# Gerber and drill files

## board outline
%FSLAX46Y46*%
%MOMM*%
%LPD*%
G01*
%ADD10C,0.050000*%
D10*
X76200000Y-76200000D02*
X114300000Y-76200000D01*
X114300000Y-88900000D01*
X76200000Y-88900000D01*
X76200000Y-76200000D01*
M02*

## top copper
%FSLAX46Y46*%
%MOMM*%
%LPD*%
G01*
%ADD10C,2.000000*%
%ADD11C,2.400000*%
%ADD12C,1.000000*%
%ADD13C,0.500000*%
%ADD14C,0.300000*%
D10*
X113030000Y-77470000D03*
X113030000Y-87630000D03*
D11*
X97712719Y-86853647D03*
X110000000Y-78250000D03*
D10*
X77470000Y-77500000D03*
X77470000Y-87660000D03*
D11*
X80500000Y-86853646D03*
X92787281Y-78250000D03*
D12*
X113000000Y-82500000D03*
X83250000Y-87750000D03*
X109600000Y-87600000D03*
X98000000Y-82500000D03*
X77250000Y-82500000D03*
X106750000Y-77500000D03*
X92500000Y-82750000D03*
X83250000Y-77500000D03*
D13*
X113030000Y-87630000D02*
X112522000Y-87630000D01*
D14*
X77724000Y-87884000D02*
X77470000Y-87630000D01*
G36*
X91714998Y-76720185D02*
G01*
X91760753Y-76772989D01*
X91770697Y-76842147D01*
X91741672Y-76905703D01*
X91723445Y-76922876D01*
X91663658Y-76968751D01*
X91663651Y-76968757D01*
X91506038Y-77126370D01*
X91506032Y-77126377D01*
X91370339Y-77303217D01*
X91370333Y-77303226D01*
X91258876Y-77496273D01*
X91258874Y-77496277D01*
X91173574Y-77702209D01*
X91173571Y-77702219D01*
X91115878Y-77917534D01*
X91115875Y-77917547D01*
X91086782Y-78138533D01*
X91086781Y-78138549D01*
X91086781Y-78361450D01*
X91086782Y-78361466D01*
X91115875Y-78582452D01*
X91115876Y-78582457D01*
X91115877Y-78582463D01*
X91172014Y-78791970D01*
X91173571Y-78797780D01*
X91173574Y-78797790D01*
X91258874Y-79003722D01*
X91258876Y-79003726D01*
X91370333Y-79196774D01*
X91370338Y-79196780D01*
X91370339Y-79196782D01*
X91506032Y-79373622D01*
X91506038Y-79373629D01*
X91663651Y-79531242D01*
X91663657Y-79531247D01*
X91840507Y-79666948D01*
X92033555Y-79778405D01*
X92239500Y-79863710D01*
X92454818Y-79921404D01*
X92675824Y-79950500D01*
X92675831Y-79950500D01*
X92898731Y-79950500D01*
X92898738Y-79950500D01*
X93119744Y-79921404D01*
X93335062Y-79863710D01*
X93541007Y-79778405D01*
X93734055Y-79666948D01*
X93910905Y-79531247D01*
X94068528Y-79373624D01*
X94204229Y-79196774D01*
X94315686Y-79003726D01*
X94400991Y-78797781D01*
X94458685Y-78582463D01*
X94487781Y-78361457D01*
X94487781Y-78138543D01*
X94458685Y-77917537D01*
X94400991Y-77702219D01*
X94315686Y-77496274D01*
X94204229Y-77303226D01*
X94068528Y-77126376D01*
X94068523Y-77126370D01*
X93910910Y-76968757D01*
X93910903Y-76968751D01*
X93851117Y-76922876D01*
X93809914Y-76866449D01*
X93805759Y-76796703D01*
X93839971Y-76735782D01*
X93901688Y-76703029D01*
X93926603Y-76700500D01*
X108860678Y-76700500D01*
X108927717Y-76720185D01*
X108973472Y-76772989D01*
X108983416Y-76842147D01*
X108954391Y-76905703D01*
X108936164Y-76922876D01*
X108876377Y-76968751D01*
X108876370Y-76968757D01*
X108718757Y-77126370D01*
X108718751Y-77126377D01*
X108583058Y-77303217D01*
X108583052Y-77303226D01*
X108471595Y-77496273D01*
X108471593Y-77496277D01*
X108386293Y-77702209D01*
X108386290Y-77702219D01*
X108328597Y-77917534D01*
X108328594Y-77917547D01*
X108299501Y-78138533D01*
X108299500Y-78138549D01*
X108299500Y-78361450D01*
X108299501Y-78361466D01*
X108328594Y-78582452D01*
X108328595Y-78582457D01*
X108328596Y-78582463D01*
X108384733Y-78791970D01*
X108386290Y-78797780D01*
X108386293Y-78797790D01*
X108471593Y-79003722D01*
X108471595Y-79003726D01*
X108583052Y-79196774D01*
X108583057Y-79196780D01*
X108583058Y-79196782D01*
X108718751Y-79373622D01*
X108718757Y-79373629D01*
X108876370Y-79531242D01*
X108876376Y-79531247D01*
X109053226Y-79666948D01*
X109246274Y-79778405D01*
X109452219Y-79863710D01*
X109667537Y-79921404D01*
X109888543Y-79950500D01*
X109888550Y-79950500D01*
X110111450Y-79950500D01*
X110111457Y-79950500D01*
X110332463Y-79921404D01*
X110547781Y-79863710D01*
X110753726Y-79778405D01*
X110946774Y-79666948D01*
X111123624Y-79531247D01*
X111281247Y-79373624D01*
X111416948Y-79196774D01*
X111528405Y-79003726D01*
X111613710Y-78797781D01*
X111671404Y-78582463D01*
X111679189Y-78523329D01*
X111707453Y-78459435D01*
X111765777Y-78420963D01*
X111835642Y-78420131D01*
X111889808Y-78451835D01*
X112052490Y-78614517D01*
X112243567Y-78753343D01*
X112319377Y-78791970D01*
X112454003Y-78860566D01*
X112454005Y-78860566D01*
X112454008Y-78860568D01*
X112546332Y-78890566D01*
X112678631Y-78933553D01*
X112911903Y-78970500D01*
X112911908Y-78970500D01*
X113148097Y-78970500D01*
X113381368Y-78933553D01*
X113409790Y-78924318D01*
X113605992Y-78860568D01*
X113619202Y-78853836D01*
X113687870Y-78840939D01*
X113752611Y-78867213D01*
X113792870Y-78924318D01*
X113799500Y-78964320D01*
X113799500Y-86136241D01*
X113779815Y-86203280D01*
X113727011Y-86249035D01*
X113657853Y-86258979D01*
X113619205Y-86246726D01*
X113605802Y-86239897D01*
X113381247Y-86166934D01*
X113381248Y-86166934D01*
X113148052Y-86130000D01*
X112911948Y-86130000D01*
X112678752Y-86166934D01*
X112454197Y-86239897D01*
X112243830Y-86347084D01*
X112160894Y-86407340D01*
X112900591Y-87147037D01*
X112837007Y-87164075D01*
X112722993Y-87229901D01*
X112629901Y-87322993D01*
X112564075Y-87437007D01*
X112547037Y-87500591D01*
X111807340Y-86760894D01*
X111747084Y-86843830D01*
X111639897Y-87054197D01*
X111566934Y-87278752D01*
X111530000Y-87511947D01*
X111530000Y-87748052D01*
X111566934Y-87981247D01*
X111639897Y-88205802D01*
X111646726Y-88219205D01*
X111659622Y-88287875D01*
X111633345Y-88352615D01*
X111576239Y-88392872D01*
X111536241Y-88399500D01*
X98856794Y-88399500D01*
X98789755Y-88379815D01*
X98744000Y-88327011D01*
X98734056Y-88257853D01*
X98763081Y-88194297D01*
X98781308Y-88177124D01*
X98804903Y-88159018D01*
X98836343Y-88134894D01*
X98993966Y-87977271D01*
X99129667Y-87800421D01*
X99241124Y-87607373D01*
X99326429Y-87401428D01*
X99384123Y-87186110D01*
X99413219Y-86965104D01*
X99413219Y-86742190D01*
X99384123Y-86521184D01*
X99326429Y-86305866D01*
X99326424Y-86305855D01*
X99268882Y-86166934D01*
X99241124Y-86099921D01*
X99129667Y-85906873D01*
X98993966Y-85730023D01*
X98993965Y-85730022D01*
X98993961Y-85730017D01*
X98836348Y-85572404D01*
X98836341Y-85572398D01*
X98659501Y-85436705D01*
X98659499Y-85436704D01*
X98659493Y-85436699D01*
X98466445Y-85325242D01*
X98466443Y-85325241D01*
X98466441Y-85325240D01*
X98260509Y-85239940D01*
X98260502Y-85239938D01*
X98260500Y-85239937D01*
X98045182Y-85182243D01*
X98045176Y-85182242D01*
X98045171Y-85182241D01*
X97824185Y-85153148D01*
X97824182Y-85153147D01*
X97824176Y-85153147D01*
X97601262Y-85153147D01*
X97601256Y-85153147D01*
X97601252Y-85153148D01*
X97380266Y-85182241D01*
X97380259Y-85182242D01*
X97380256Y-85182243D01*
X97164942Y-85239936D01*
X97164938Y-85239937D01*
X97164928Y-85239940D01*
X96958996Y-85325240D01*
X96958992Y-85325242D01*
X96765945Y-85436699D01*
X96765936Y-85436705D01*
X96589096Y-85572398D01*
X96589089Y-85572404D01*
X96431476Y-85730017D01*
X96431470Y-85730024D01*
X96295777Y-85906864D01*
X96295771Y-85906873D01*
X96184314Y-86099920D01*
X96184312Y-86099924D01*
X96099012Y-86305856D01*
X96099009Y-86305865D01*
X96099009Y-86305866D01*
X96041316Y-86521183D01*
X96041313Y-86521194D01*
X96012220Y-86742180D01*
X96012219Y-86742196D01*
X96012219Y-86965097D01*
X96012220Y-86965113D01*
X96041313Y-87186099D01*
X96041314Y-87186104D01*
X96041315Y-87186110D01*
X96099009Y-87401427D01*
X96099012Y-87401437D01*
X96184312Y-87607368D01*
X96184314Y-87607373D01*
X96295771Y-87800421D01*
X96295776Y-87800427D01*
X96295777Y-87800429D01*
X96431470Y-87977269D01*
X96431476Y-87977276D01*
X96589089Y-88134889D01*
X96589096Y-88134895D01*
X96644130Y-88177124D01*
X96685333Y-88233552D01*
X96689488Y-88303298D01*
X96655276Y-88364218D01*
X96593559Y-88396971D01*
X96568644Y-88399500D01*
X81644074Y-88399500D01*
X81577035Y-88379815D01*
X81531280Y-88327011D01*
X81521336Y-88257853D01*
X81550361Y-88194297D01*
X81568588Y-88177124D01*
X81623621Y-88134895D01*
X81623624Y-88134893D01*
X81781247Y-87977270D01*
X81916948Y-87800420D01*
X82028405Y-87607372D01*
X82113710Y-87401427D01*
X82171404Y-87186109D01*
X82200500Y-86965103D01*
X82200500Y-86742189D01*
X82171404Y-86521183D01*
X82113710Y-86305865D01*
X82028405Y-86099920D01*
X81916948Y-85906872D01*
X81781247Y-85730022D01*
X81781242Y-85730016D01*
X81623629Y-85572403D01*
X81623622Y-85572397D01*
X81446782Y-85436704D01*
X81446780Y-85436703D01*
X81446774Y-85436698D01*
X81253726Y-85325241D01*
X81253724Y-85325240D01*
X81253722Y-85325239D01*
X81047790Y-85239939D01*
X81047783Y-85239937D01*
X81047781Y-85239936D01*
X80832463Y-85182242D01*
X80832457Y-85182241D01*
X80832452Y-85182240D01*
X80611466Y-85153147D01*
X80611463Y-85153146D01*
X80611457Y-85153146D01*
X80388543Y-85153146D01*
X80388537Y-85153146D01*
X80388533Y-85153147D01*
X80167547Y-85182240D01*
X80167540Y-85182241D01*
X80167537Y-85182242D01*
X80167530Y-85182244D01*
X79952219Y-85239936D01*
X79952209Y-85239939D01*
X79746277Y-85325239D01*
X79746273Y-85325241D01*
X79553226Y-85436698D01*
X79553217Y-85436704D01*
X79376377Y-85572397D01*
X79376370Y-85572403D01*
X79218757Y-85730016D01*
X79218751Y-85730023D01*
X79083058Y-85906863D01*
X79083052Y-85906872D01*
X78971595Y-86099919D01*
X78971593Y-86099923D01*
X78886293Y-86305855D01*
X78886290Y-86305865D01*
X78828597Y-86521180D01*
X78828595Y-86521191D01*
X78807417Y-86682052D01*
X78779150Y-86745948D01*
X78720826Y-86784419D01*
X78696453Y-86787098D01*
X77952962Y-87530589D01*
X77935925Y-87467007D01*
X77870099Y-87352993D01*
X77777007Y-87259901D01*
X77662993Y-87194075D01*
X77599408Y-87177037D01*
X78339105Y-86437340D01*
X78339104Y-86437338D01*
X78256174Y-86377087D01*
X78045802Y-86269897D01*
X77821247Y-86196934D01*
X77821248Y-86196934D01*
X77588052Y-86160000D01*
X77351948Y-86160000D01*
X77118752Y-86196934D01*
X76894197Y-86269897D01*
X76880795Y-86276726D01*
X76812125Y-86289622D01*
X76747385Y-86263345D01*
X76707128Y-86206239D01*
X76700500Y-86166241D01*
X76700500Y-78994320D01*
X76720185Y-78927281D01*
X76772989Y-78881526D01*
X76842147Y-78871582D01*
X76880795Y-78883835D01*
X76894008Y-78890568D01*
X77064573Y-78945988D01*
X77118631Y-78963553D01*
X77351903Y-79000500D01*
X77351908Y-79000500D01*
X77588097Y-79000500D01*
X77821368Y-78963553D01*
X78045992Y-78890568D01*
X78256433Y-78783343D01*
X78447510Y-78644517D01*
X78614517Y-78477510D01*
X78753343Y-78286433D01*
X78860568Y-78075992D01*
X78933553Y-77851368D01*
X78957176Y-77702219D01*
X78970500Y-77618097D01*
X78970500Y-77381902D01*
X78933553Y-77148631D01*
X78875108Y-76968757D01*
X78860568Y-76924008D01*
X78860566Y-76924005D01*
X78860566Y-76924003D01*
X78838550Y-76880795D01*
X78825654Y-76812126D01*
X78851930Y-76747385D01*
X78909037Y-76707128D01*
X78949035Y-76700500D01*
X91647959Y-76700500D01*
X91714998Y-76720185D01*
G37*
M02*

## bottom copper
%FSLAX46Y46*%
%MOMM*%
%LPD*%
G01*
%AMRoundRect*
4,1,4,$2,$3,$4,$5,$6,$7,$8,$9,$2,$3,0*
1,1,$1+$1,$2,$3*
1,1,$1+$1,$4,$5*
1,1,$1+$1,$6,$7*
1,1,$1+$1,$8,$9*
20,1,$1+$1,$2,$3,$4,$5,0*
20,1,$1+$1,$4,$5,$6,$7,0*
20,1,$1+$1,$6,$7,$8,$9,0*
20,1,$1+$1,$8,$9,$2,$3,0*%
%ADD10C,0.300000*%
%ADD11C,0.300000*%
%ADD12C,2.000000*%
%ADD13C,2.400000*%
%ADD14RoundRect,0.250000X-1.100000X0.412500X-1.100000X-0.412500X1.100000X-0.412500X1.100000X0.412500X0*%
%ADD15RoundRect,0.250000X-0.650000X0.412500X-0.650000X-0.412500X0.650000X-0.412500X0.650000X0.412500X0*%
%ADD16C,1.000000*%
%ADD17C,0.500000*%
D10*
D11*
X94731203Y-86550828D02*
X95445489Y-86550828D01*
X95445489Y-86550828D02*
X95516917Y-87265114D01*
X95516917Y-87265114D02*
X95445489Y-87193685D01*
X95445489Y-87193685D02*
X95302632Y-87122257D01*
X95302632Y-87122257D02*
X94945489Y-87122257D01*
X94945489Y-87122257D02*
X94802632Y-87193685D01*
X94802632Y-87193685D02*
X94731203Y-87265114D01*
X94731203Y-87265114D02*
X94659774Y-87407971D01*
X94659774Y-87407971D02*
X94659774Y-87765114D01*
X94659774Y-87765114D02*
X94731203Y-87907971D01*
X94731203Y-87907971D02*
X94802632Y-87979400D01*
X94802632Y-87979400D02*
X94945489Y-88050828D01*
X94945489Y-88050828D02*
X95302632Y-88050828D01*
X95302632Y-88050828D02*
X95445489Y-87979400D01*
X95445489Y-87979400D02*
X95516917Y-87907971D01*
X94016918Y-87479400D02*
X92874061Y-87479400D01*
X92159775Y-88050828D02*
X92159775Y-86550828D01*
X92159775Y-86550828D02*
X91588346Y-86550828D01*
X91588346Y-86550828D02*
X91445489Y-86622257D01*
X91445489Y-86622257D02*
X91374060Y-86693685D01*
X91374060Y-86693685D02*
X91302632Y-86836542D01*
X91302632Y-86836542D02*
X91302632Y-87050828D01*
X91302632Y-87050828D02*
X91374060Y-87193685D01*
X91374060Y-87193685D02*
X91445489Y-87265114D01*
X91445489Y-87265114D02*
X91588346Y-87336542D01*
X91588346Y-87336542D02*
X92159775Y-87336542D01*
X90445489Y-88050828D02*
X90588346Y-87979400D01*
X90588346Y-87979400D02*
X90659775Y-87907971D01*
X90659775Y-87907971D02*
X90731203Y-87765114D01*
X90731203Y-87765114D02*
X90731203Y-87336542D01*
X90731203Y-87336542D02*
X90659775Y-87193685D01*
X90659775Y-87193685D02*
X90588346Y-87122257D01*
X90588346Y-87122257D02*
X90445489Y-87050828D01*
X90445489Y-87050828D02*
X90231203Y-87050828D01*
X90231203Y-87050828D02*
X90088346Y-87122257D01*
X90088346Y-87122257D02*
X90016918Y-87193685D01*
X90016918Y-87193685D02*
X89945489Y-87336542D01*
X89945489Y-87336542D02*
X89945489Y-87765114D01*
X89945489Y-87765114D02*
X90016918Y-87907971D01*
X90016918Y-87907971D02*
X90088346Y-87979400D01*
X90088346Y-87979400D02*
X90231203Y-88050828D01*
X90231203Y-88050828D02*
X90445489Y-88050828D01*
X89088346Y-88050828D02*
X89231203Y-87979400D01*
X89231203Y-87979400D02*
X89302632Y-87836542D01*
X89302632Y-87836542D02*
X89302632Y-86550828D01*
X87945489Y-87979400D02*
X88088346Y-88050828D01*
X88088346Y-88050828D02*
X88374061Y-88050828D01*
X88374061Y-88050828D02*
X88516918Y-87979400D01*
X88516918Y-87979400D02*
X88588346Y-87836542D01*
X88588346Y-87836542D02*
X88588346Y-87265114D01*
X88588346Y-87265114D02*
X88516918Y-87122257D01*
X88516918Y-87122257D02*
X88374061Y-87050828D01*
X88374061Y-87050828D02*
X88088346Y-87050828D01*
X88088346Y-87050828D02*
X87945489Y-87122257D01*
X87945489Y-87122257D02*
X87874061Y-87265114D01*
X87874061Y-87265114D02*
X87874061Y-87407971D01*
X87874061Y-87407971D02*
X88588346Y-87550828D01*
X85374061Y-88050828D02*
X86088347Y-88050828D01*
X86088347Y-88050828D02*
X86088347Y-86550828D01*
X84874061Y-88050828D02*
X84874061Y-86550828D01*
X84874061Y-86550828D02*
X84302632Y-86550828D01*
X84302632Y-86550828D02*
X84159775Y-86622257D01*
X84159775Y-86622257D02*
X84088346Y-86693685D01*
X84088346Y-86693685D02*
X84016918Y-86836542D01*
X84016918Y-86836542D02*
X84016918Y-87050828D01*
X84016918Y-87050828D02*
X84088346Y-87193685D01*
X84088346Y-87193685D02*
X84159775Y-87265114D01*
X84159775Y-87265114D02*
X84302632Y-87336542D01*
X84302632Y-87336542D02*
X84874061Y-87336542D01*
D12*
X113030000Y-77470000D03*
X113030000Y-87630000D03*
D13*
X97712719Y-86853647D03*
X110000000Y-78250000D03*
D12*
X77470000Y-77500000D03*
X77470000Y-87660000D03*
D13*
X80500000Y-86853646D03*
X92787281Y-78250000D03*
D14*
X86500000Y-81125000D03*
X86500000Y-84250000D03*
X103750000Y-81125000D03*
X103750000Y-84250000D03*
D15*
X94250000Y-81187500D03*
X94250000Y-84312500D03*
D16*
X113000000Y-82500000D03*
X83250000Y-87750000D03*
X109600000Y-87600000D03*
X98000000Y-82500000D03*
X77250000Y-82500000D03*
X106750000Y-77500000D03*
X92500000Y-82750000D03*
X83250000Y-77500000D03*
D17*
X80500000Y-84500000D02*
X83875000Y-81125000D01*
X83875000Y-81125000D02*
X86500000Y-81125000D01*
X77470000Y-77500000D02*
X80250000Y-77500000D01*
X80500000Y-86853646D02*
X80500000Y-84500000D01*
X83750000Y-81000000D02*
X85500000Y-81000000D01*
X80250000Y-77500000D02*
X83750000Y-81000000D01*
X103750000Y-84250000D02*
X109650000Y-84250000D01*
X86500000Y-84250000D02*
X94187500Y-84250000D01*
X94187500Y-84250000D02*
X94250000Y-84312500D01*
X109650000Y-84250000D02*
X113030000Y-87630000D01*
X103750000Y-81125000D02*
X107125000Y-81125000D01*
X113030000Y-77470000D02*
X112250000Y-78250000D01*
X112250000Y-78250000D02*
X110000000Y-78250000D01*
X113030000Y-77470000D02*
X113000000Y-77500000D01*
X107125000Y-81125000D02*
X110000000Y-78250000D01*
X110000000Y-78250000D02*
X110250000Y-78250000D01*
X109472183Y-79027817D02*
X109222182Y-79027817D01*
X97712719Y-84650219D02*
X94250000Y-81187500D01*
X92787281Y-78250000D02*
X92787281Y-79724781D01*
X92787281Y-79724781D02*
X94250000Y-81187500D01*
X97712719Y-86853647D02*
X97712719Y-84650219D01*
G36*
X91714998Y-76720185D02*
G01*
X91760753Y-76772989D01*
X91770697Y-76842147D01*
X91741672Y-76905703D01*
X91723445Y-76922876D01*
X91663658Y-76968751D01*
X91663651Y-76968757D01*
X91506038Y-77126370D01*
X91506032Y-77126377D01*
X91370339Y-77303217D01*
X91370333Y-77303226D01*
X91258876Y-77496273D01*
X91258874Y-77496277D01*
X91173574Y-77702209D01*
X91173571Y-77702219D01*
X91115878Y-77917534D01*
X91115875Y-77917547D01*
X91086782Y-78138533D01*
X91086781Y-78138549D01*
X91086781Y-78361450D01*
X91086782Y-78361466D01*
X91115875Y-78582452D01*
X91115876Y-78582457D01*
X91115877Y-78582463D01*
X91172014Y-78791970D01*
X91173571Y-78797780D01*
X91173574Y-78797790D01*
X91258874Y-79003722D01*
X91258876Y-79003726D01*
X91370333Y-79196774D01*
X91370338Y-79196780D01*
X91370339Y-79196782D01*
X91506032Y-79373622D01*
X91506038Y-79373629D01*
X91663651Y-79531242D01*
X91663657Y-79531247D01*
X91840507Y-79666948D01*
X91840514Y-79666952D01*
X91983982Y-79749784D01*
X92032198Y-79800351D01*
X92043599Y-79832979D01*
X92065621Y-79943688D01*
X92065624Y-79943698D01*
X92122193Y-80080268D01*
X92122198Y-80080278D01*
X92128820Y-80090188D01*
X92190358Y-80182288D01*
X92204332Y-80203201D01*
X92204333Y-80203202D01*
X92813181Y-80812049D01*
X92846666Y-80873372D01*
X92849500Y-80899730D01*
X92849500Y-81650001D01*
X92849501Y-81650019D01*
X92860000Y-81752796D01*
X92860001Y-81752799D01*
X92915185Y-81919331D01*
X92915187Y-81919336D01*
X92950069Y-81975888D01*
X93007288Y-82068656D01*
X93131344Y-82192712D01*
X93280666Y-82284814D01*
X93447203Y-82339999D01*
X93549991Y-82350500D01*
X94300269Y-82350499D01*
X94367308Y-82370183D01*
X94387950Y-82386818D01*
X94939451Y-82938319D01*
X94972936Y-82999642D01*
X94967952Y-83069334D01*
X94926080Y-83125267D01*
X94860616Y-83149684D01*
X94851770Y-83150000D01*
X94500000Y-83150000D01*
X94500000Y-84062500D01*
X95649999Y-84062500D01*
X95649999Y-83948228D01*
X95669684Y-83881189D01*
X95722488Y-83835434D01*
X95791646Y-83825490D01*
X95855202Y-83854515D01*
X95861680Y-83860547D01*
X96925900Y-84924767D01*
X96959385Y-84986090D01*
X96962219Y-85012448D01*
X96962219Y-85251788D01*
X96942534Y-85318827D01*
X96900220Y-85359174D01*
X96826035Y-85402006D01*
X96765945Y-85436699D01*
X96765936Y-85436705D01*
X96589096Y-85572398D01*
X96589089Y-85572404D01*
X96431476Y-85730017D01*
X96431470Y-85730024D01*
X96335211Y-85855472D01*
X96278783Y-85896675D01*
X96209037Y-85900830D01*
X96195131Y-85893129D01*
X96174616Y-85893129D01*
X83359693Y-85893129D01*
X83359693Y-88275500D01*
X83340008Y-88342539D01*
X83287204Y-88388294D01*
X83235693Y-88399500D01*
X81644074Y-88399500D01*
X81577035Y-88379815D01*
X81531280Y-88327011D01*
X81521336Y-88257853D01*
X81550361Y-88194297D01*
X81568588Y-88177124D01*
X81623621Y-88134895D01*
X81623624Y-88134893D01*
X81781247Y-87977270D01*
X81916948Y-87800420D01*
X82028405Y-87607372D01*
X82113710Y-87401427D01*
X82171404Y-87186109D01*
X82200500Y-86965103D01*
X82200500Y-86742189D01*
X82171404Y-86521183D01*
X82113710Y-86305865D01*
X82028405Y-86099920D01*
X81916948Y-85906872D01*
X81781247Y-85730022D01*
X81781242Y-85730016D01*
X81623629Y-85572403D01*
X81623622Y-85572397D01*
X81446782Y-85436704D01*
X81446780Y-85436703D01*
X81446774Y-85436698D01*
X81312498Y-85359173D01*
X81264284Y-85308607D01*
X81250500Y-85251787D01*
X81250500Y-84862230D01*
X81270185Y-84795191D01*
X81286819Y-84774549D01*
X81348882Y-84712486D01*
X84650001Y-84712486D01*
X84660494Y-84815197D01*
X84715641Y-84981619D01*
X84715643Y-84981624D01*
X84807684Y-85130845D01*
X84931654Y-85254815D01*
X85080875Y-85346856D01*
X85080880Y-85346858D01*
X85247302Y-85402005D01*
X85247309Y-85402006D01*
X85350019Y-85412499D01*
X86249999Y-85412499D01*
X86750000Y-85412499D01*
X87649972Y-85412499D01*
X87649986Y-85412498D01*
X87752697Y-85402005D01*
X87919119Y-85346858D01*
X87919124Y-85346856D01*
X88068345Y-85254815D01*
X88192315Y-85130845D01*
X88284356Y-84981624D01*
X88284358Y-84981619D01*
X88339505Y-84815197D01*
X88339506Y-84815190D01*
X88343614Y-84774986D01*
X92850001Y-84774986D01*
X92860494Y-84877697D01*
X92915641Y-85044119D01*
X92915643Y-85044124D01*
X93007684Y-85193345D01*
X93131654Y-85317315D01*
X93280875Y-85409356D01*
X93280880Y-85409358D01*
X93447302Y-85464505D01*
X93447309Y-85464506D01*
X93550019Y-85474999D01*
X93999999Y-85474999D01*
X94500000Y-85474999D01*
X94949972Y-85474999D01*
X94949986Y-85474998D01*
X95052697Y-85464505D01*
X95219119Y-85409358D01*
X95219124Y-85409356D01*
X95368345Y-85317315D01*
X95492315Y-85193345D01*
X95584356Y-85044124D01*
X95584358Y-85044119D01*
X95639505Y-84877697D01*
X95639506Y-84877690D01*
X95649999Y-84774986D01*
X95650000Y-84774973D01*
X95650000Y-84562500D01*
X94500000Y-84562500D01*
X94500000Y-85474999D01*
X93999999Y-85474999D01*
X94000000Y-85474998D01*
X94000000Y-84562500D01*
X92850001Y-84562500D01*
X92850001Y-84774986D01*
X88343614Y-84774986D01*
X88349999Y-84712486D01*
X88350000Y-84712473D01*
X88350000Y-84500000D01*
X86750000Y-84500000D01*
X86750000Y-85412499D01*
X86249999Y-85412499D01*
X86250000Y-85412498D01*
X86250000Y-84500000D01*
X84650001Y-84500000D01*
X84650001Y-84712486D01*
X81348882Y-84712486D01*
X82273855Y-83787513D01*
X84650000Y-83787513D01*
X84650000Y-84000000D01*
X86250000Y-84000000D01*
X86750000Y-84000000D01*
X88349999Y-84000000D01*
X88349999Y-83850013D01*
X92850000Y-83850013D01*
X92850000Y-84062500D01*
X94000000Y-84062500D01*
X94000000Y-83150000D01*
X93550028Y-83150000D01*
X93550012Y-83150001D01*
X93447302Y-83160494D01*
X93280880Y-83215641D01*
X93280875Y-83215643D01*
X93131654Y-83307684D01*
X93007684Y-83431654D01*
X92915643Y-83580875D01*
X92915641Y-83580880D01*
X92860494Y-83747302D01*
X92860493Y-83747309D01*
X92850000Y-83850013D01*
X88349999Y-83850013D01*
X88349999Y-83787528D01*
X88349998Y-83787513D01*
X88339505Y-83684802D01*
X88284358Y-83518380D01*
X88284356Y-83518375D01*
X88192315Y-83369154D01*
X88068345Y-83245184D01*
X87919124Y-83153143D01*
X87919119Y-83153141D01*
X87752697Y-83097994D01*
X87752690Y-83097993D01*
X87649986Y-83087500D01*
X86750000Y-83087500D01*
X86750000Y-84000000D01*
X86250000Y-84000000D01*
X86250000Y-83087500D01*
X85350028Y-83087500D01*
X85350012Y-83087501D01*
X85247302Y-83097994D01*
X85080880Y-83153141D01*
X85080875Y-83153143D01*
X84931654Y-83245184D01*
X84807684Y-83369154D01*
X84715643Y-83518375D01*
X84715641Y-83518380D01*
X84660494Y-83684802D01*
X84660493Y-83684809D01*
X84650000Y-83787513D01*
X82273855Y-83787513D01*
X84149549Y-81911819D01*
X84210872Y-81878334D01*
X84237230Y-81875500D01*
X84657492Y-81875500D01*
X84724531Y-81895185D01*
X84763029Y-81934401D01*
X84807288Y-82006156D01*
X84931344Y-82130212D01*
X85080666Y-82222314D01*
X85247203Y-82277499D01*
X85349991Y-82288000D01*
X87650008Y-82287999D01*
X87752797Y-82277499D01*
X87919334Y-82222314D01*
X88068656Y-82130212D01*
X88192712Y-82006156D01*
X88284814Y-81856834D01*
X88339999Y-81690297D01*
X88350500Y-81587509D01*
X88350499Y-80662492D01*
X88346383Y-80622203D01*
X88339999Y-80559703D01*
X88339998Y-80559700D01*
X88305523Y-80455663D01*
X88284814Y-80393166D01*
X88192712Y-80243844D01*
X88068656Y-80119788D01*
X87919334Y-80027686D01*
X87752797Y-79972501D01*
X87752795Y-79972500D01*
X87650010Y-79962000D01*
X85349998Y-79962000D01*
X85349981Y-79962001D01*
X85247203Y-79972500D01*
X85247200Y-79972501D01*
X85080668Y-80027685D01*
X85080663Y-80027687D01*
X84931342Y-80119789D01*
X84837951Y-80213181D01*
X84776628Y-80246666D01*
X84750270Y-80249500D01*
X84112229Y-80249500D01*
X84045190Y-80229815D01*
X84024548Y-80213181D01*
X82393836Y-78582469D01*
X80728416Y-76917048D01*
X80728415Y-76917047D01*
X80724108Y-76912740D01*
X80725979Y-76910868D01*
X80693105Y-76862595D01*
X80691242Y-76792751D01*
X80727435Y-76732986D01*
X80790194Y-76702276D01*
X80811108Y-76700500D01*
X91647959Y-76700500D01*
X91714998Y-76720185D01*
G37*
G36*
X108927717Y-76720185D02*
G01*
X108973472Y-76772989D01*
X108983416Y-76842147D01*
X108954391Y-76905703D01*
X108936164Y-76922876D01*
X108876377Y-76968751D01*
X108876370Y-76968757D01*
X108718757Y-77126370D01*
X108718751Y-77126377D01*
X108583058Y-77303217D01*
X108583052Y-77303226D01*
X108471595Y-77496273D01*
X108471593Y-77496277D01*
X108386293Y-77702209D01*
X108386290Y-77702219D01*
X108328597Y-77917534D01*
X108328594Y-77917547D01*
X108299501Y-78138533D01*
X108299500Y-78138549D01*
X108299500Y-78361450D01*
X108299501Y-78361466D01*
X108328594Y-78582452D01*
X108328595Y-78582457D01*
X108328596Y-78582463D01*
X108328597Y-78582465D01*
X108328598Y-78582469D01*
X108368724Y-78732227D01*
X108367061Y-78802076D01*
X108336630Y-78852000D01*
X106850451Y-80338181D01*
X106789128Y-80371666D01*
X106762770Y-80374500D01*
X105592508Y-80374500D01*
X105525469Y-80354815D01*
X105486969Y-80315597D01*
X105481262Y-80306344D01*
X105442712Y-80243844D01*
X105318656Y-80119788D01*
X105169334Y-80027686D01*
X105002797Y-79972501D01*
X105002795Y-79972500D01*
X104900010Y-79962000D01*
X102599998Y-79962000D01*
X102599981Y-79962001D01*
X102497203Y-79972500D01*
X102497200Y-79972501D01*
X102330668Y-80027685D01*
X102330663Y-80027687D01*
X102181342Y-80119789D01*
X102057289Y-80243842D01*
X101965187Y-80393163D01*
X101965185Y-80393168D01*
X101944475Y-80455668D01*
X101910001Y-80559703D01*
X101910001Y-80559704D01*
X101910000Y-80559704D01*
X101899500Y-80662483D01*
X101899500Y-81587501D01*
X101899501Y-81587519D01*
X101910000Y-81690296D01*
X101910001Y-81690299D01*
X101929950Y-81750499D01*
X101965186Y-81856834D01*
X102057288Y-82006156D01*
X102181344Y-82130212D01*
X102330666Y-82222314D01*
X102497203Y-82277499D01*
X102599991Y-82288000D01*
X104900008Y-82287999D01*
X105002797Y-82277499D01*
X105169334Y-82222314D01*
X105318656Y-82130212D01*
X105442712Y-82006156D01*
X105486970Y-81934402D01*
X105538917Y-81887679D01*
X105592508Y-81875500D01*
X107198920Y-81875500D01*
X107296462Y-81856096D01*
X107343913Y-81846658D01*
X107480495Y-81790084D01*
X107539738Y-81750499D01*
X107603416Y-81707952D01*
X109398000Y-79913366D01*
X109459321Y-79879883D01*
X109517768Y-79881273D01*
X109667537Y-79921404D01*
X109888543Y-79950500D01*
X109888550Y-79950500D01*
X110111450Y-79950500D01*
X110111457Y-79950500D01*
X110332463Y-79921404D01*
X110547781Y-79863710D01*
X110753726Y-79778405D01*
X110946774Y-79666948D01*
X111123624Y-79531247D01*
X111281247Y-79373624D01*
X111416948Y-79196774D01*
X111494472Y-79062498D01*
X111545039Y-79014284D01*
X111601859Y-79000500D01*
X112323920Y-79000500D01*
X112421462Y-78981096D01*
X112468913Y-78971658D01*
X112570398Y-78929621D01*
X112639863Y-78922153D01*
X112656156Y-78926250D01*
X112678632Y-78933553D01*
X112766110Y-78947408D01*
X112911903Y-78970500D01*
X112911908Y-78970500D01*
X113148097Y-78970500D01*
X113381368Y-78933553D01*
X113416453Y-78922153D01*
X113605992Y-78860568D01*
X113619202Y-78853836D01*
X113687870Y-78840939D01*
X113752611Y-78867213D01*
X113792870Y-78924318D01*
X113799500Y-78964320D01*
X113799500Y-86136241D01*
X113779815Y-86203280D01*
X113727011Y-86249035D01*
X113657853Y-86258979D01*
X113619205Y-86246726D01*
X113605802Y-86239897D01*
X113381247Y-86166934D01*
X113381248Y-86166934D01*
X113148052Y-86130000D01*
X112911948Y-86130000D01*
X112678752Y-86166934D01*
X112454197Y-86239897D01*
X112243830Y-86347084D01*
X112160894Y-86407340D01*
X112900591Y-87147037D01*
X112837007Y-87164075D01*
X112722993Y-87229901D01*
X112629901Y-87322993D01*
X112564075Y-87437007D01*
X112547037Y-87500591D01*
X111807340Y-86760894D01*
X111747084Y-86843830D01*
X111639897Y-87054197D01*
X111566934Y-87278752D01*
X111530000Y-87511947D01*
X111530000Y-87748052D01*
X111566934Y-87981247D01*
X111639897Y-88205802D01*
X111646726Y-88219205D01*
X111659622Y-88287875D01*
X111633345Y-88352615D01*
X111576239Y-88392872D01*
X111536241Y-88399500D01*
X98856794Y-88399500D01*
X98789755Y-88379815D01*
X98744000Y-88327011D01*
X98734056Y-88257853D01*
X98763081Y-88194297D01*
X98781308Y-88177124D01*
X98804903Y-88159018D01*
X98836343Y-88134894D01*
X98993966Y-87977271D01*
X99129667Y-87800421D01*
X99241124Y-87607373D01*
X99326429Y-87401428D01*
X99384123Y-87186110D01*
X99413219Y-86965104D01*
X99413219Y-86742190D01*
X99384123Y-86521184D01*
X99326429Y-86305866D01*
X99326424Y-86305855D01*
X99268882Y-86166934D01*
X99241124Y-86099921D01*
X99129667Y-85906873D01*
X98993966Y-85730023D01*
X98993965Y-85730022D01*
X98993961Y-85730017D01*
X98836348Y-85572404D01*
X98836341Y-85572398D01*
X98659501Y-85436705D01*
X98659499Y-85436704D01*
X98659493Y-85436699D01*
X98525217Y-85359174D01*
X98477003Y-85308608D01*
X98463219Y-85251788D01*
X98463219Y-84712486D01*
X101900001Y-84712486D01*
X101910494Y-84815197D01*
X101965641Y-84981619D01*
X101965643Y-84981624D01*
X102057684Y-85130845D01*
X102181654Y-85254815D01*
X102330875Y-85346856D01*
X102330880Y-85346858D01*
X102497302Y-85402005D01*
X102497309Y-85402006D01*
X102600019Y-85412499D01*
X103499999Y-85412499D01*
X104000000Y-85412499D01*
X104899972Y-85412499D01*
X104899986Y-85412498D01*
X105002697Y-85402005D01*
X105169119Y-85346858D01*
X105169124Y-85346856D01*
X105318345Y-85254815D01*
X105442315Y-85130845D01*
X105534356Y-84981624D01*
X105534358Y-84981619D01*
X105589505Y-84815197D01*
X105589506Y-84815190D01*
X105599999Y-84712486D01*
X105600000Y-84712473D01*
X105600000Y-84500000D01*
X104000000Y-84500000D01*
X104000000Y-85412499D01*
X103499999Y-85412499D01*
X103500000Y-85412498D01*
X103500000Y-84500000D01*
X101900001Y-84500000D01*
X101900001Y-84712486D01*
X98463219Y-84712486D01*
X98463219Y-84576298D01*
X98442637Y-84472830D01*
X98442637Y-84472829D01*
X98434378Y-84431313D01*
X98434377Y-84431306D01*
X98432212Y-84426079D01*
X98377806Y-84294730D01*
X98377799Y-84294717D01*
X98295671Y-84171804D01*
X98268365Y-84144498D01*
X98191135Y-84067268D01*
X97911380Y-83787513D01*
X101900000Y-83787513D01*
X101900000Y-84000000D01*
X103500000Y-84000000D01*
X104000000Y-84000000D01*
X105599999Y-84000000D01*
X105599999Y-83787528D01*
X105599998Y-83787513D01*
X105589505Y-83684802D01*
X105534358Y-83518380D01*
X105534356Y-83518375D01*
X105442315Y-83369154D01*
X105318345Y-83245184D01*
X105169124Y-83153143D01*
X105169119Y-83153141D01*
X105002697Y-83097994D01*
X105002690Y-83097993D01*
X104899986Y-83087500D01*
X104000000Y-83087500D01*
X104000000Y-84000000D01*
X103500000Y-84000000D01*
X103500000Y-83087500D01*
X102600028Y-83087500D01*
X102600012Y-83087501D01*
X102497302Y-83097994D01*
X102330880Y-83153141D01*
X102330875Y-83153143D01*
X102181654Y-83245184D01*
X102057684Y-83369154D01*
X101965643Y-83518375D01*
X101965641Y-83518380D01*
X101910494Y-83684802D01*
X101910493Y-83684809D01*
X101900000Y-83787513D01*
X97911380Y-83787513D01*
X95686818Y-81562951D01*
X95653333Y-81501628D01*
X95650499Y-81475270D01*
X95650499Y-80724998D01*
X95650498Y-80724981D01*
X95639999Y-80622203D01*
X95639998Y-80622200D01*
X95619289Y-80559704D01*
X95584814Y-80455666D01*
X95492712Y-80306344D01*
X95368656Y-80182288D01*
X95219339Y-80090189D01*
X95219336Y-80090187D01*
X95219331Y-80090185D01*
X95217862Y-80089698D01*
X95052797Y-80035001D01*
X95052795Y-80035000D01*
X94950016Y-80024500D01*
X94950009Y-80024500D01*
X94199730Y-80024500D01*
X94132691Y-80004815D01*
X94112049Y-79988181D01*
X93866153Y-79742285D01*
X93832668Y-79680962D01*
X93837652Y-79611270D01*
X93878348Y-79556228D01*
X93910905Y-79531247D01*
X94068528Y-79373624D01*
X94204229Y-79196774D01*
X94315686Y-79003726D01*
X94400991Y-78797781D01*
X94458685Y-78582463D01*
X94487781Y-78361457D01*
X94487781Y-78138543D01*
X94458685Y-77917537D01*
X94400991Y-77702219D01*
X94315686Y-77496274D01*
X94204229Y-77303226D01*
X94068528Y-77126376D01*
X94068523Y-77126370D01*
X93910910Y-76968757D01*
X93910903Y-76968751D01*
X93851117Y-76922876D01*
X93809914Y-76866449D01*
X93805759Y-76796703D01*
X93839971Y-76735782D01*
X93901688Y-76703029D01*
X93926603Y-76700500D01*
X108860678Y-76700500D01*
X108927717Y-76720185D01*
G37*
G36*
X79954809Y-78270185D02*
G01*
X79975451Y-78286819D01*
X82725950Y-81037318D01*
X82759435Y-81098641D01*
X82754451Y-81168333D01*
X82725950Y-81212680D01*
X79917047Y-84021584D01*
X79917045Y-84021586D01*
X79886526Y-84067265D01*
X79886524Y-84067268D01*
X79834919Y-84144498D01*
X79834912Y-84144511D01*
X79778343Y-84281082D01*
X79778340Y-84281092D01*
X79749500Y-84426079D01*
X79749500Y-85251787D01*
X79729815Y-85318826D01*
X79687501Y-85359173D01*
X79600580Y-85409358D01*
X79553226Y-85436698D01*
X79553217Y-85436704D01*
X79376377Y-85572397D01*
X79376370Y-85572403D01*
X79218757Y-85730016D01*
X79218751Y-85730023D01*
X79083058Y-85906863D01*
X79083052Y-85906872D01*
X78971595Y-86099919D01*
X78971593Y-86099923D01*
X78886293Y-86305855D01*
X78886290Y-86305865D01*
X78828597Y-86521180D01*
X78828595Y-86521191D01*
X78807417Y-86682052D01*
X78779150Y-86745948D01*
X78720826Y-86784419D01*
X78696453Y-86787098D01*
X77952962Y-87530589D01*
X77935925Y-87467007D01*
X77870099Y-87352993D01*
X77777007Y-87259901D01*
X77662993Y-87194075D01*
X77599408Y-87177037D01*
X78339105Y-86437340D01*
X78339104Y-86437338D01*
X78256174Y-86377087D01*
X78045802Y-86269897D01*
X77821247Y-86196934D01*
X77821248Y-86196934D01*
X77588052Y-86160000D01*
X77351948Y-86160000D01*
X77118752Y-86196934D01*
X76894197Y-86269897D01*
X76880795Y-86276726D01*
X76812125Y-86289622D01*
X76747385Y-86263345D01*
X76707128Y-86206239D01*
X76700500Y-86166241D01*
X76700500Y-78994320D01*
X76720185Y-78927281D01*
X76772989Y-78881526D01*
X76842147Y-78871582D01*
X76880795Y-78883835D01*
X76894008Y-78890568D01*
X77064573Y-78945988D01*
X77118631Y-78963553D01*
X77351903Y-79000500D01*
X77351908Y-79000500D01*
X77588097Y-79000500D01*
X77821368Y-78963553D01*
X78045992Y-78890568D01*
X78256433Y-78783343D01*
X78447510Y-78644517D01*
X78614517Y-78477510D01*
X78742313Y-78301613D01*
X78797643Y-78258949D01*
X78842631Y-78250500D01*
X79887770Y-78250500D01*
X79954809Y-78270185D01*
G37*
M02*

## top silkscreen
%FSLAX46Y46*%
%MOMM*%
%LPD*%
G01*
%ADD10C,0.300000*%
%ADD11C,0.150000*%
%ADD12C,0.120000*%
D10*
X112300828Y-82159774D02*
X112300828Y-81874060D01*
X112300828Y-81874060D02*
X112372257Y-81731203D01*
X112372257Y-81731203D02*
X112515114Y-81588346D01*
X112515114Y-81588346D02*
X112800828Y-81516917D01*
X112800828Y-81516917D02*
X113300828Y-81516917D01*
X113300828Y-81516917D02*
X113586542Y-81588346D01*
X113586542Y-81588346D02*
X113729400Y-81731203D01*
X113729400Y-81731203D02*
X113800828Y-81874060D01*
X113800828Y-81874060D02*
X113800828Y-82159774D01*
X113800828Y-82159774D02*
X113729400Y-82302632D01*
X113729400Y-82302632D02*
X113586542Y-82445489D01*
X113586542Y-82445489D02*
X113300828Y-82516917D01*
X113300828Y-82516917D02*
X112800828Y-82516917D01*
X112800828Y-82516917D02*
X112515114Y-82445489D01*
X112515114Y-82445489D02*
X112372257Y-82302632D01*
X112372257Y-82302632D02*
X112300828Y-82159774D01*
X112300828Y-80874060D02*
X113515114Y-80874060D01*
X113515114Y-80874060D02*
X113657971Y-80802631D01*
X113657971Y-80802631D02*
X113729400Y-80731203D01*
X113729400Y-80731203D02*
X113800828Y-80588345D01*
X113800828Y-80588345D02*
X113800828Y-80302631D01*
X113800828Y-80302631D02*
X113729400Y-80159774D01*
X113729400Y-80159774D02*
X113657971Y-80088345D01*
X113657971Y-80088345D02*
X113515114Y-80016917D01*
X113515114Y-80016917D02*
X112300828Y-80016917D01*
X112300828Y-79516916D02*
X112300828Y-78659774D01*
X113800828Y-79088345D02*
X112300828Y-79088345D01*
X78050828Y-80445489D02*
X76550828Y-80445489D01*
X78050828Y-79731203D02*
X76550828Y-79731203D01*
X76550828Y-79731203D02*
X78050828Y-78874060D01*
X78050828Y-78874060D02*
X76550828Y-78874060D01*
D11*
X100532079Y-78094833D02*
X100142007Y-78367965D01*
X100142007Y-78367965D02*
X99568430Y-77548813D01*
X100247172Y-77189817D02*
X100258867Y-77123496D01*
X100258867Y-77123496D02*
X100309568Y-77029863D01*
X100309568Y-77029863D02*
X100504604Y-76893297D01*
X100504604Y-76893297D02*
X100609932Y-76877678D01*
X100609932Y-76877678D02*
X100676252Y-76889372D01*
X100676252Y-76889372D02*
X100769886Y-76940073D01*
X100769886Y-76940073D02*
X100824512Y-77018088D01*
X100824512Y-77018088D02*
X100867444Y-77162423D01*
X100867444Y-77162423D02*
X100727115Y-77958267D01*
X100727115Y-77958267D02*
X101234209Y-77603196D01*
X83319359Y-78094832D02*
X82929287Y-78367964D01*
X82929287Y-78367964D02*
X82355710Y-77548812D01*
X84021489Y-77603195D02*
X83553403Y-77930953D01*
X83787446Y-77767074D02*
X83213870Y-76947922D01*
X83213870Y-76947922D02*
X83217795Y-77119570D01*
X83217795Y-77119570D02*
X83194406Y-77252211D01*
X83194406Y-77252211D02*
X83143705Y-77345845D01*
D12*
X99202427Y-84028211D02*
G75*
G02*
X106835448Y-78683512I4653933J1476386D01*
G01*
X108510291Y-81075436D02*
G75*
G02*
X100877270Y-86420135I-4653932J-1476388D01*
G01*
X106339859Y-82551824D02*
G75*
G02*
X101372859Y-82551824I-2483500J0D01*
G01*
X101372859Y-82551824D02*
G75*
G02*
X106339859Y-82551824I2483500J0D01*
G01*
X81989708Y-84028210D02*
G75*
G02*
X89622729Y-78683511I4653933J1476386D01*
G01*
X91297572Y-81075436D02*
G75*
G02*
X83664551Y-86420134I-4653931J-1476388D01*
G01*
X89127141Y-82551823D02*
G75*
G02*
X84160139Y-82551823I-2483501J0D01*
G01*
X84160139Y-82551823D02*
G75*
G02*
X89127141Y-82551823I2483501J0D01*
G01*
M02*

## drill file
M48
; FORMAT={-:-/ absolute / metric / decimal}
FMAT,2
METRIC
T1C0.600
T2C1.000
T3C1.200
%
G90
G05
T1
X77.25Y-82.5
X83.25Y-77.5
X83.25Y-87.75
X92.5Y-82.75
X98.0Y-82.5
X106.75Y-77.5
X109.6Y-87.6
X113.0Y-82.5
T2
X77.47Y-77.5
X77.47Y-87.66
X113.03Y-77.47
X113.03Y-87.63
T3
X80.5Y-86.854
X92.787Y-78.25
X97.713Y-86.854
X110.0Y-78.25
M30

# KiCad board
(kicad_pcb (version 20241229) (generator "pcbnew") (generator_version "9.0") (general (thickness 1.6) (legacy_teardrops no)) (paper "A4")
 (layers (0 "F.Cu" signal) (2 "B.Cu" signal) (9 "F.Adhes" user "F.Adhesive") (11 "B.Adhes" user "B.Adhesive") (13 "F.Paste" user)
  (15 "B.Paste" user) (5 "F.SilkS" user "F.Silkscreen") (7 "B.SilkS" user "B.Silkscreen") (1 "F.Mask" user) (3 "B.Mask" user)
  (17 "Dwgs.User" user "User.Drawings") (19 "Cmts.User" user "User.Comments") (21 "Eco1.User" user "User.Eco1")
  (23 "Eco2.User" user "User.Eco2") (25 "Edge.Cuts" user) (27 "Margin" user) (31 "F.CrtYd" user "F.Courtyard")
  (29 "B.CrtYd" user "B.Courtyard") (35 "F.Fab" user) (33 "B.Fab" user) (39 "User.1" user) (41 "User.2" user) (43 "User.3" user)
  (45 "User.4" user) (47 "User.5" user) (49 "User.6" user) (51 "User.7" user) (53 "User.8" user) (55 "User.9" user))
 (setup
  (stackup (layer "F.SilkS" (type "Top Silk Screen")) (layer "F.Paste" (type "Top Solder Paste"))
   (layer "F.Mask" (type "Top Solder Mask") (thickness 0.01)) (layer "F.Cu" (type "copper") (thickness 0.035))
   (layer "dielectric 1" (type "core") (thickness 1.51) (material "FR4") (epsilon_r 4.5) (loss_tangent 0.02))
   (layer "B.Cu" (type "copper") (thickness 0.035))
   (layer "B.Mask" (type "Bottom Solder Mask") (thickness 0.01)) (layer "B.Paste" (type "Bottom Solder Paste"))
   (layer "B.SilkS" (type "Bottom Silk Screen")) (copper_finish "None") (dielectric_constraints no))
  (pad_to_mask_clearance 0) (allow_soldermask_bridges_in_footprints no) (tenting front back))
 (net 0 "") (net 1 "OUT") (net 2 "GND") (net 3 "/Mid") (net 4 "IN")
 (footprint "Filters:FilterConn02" (layer "F.Cu") (at 113.03 82.55)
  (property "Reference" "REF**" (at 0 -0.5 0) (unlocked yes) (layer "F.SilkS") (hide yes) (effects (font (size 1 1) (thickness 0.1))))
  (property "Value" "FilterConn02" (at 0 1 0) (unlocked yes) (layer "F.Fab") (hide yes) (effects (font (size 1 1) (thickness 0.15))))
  (pad "3" thru_hole circle (at 0 -5.08) (size 2 2) (drill 1) (layers "*.Cu" "*.Mask") (remove_unused_layers no) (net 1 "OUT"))
  (pad "4" thru_hole circle (at 0 5.08) (size 2 2) (drill 1) (layers "*.Cu" "*.Mask") (remove_unused_layers no) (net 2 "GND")))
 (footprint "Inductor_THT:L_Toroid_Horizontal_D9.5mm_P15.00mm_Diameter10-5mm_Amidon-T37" (layer "F.Cu") (at 97.712719 86.853647 35)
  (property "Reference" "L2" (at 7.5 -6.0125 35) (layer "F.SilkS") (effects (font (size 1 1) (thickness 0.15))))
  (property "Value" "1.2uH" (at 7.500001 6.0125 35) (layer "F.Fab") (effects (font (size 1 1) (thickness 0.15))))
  (fp_arc (start 2.840901 -1.46) (mid 7.5 -4.882499) (end 12.159099 -1.46) (stroke (width 0.12) (type solid)) (layer "F.SilkS"))
  (fp_arc (start 12.159099 1.46) (mid 7.5 4.8825) (end 2.840901 1.46) (stroke (width 0.12) (type solid)) (layer "F.SilkS"))
  (fp_circle (center 7.5 0) (end 9.983499 0) (stroke (width 0.12) (type solid)) (fill no) (layer "F.SilkS"))
  (pad "1" thru_hole circle (at 0 0 35) (size 2.4 2.4) (drill 1.2) (layers "*.Cu" "*.Mask") (remove_unused_layers no) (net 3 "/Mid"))
  (pad "2" thru_hole circle (at 15.000001 0 35) (size 2.4 2.4) (drill 1.2) (layers "*.Cu" "*.Mask") (remove_unused_layers no)))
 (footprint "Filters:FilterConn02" (layer "F.Cu") (at 77.47 82.58)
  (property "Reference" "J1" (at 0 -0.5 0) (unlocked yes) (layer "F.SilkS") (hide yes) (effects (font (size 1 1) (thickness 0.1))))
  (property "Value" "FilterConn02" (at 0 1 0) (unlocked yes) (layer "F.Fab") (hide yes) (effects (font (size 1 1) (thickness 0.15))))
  (pad "1" thru_hole circle (at 0 -5.08) (size 2 2) (drill 1) (layers "*.Cu" "*.Mask") (remove_unused_layers no) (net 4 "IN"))
  (pad "2" thru_hole circle (at 0 5.08) (size 2 2) (drill 1) (layers "*.Cu" "*.Mask") (remove_unused_layers no) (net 2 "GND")))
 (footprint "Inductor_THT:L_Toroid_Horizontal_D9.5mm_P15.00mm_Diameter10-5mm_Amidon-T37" (layer "F.Cu") (at 80.5 86.853646 35)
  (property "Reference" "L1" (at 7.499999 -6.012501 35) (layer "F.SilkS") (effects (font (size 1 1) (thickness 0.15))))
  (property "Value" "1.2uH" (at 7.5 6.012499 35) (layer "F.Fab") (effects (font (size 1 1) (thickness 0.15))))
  (fp_arc (start 2.840901 -1.46) (mid 7.5 -4.882499) (end 12.159099 -1.46) (stroke (width 0.12) (type solid)) (layer "F.SilkS"))
  (fp_arc (start 12.159098 1.46) (mid 7.5 4.8825) (end 2.840901 1.46) (stroke (width 0.12) (type solid)) (layer "F.SilkS"))
  (fp_circle (center 7.5 0) (end 9.983501 0) (stroke (width 0.12) (type solid)) (fill no) (layer "F.SilkS"))
  (pad "1" thru_hole circle (at 0 0 35) (size 2.4 2.4) (drill 1.2) (layers "*.Cu" "*.Mask") (remove_unused_layers no))
  (pad "2" thru_hole circle (at 15 0.000001 35) (size 2.4 2.4) (drill 1.2) (layers "*.Cu" "*.Mask") (remove_unused_layers no) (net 3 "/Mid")))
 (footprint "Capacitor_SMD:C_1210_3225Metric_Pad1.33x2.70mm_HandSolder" (layer "B.Cu") (at 86.5 82.6875 -90)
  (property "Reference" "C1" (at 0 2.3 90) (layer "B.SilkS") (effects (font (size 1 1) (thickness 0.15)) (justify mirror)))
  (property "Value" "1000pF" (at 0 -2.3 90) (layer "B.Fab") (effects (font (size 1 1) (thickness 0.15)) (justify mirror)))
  (pad "1" smd roundrect (at -1.5625 0 270) (size 1.325 2.7) (layers "B.Cu" "B.Mask" "B.Paste") (roundrect_rratio 0.188679))
  (pad "2" smd roundrect (at 1.5625 0 270) (size 1.325 2.7) (layers "B.Cu" "B.Mask" "B.Paste") (roundrect_rratio 0.188679) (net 2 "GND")))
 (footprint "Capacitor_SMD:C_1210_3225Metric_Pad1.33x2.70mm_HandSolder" (layer "B.Cu") (at 103.75 82.6875 -90)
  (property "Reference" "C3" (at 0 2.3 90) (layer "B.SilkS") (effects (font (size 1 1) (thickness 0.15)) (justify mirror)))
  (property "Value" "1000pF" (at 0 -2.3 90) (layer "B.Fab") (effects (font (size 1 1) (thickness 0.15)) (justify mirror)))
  (pad "1" smd roundrect (at -1.5625 0 270) (size 1.325 2.7) (layers "B.Cu" "B.Mask" "B.Paste") (roundrect_rratio 0.188679))
  (pad "2" smd roundrect (at 1.5625 0 270) (size 1.325 2.7) (layers "B.Cu" "B.Mask" "B.Paste") (roundrect_rratio 0.188679) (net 2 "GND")))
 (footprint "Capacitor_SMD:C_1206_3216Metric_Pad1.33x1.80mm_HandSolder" (layer "B.Cu") (at 94.25 82.75 -90)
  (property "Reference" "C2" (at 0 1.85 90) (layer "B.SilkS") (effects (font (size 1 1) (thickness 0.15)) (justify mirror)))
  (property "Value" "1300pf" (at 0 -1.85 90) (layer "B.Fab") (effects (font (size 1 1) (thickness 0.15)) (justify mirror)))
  (pad "1" smd roundrect (at -1.5625 0 270) (size 1.325 1.8) (layers "B.Cu" "B.Mask" "B.Paste") (roundrect_rratio 0.188679) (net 3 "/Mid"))
  (pad "2" smd roundrect (at 1.5625 0 270) (size 1.325 1.8) (layers "B.Cu" "B.Mask" "B.Paste") (roundrect_rratio 0.188679) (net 2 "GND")))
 (gr_rect (start 76.2 76.2) (end 114.3 88.9) (stroke (width 0.05) (type default)) (fill no) (layer "Edge.Cuts"))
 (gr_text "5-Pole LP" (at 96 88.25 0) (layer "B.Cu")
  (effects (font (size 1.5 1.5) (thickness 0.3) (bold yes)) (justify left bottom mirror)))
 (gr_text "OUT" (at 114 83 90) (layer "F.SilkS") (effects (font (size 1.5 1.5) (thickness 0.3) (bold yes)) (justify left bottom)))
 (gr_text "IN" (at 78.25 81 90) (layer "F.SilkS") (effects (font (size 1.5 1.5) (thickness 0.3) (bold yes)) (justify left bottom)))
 (segment (start 80.5 84.5) (end 83.875 81.125) (width 0.5) (layer "B.Cu") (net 4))
 (segment (start 83.875 81.125) (end 86.5 81.125) (width 0.5) (layer "B.Cu") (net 4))
 (segment (start 77.47 77.5) (end 80.25 77.5) (width 0.5) (layer "B.Cu") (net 4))
 (segment (start 80.5 86.853646) (end 80.5 84.5) (width 0.5) (layer "B.Cu") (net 4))
 (segment (start 83.75 81) (end 85.5 81) (width 0.5) (layer "B.Cu") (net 4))
 (segment (start 80.25 77.5) (end 83.75 81) (width 0.5) (layer "B.Cu") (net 4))
 (segment (start 113.03 87.63) (end 112.522 87.63) (width 0.5) (layer "F.Cu") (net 2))
 (segment (start 77.724 87.884) (end 77.47 87.63) (width 0.3) (layer "F.Cu") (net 2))
 (via (at 113 82.5) (size 1) (drill 0.6) (layers "F.Cu" "B.Cu") (free yes) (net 2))
 (via (at 83.25 87.75) (size 1) (drill 0.6) (layers "F.Cu" "B.Cu") (free yes) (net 2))
 (via (at 109.6 87.6) (size 1) (drill 0.6) (layers "F.Cu" "B.Cu") (free yes) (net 2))
 (via (at 98 82.5) (size 1) (drill 0.6) (layers "F.Cu" "B.Cu") (free yes) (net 2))
 (via (at 77.25 82.5) (size 1) (drill 0.6) (layers "F.Cu" "B.Cu") (free yes) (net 2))
 (via (at 106.75 77.5) (size 1) (drill 0.6) (layers "F.Cu" "B.Cu") (free yes) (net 2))
 (via (at 92.5 82.75) (size 1) (drill 0.6) (layers "F.Cu" "B.Cu") (free yes) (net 2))
 (via (at 83.25 77.5) (size 1) (drill 0.6) (layers "F.Cu" "B.Cu") (free yes) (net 2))
 (segment (start 103.75 84.25) (end 109.65 84.25) (width 0.5) (layer "B.Cu") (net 2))
 (segment (start 86.5 84.25) (end 94.1875 84.25) (width 0.5) (layer "B.Cu") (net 2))
 (segment (start 94.1875 84.25) (end 94.25 84.3125) (width 0.5) (layer "B.Cu") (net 2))
 (segment (start 109.65 84.25) (end 113.03 87.63) (width 0.5) (layer "B.Cu") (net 2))
 (segment (start 103.75 81.125) (end 107.125 81.125) (width 0.5) (layer "B.Cu") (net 1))
 (segment (start 113.03 77.47) (end 112.25 78.25) (width 0.5) (layer "B.Cu") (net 1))
 (segment (start 112.25 78.25) (end 110 78.25) (width 0.5) (layer "B.Cu") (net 1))
 (segment (start 113.03 77.47) (end 113 77.5) (width 0.5) (layer "B.Cu") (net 1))
 (segment (start 107.125 81.125) (end 110 78.25) (width 0.5) (layer "B.Cu") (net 1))
 (segment (start 110 78.25) (end 110.25 78.25) (width 0.5) (layer "B.Cu") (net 1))
 (segment (start 109.472183 79.027817) (end 109.222182 79.027817) (width 0.5) (layer "B.Cu") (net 1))
 (segment (start 97.712719 84.650219) (end 94.25 81.1875) (width 0.5) (layer "B.Cu") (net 3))
 (segment (start 92.787281 78.25) (end 92.787281 79.724781) (width 0.5) (layer "B.Cu") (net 3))
 (segment (start 92.787281 79.724781) (end 94.25 81.1875) (width 0.5) (layer "B.Cu") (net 3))
 (segment (start 97.712719 86.853647) (end 97.712719 84.650219) (width 0.5) (layer "B.Cu") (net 3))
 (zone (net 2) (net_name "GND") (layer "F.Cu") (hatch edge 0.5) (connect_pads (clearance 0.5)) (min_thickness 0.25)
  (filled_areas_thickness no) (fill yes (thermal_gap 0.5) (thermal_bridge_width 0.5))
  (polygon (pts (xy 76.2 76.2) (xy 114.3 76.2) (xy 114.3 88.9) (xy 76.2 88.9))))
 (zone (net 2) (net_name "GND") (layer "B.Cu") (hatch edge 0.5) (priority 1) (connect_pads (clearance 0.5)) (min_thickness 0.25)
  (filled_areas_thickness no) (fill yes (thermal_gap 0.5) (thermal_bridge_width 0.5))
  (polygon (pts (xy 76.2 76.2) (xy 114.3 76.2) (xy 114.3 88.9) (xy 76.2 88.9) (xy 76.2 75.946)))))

